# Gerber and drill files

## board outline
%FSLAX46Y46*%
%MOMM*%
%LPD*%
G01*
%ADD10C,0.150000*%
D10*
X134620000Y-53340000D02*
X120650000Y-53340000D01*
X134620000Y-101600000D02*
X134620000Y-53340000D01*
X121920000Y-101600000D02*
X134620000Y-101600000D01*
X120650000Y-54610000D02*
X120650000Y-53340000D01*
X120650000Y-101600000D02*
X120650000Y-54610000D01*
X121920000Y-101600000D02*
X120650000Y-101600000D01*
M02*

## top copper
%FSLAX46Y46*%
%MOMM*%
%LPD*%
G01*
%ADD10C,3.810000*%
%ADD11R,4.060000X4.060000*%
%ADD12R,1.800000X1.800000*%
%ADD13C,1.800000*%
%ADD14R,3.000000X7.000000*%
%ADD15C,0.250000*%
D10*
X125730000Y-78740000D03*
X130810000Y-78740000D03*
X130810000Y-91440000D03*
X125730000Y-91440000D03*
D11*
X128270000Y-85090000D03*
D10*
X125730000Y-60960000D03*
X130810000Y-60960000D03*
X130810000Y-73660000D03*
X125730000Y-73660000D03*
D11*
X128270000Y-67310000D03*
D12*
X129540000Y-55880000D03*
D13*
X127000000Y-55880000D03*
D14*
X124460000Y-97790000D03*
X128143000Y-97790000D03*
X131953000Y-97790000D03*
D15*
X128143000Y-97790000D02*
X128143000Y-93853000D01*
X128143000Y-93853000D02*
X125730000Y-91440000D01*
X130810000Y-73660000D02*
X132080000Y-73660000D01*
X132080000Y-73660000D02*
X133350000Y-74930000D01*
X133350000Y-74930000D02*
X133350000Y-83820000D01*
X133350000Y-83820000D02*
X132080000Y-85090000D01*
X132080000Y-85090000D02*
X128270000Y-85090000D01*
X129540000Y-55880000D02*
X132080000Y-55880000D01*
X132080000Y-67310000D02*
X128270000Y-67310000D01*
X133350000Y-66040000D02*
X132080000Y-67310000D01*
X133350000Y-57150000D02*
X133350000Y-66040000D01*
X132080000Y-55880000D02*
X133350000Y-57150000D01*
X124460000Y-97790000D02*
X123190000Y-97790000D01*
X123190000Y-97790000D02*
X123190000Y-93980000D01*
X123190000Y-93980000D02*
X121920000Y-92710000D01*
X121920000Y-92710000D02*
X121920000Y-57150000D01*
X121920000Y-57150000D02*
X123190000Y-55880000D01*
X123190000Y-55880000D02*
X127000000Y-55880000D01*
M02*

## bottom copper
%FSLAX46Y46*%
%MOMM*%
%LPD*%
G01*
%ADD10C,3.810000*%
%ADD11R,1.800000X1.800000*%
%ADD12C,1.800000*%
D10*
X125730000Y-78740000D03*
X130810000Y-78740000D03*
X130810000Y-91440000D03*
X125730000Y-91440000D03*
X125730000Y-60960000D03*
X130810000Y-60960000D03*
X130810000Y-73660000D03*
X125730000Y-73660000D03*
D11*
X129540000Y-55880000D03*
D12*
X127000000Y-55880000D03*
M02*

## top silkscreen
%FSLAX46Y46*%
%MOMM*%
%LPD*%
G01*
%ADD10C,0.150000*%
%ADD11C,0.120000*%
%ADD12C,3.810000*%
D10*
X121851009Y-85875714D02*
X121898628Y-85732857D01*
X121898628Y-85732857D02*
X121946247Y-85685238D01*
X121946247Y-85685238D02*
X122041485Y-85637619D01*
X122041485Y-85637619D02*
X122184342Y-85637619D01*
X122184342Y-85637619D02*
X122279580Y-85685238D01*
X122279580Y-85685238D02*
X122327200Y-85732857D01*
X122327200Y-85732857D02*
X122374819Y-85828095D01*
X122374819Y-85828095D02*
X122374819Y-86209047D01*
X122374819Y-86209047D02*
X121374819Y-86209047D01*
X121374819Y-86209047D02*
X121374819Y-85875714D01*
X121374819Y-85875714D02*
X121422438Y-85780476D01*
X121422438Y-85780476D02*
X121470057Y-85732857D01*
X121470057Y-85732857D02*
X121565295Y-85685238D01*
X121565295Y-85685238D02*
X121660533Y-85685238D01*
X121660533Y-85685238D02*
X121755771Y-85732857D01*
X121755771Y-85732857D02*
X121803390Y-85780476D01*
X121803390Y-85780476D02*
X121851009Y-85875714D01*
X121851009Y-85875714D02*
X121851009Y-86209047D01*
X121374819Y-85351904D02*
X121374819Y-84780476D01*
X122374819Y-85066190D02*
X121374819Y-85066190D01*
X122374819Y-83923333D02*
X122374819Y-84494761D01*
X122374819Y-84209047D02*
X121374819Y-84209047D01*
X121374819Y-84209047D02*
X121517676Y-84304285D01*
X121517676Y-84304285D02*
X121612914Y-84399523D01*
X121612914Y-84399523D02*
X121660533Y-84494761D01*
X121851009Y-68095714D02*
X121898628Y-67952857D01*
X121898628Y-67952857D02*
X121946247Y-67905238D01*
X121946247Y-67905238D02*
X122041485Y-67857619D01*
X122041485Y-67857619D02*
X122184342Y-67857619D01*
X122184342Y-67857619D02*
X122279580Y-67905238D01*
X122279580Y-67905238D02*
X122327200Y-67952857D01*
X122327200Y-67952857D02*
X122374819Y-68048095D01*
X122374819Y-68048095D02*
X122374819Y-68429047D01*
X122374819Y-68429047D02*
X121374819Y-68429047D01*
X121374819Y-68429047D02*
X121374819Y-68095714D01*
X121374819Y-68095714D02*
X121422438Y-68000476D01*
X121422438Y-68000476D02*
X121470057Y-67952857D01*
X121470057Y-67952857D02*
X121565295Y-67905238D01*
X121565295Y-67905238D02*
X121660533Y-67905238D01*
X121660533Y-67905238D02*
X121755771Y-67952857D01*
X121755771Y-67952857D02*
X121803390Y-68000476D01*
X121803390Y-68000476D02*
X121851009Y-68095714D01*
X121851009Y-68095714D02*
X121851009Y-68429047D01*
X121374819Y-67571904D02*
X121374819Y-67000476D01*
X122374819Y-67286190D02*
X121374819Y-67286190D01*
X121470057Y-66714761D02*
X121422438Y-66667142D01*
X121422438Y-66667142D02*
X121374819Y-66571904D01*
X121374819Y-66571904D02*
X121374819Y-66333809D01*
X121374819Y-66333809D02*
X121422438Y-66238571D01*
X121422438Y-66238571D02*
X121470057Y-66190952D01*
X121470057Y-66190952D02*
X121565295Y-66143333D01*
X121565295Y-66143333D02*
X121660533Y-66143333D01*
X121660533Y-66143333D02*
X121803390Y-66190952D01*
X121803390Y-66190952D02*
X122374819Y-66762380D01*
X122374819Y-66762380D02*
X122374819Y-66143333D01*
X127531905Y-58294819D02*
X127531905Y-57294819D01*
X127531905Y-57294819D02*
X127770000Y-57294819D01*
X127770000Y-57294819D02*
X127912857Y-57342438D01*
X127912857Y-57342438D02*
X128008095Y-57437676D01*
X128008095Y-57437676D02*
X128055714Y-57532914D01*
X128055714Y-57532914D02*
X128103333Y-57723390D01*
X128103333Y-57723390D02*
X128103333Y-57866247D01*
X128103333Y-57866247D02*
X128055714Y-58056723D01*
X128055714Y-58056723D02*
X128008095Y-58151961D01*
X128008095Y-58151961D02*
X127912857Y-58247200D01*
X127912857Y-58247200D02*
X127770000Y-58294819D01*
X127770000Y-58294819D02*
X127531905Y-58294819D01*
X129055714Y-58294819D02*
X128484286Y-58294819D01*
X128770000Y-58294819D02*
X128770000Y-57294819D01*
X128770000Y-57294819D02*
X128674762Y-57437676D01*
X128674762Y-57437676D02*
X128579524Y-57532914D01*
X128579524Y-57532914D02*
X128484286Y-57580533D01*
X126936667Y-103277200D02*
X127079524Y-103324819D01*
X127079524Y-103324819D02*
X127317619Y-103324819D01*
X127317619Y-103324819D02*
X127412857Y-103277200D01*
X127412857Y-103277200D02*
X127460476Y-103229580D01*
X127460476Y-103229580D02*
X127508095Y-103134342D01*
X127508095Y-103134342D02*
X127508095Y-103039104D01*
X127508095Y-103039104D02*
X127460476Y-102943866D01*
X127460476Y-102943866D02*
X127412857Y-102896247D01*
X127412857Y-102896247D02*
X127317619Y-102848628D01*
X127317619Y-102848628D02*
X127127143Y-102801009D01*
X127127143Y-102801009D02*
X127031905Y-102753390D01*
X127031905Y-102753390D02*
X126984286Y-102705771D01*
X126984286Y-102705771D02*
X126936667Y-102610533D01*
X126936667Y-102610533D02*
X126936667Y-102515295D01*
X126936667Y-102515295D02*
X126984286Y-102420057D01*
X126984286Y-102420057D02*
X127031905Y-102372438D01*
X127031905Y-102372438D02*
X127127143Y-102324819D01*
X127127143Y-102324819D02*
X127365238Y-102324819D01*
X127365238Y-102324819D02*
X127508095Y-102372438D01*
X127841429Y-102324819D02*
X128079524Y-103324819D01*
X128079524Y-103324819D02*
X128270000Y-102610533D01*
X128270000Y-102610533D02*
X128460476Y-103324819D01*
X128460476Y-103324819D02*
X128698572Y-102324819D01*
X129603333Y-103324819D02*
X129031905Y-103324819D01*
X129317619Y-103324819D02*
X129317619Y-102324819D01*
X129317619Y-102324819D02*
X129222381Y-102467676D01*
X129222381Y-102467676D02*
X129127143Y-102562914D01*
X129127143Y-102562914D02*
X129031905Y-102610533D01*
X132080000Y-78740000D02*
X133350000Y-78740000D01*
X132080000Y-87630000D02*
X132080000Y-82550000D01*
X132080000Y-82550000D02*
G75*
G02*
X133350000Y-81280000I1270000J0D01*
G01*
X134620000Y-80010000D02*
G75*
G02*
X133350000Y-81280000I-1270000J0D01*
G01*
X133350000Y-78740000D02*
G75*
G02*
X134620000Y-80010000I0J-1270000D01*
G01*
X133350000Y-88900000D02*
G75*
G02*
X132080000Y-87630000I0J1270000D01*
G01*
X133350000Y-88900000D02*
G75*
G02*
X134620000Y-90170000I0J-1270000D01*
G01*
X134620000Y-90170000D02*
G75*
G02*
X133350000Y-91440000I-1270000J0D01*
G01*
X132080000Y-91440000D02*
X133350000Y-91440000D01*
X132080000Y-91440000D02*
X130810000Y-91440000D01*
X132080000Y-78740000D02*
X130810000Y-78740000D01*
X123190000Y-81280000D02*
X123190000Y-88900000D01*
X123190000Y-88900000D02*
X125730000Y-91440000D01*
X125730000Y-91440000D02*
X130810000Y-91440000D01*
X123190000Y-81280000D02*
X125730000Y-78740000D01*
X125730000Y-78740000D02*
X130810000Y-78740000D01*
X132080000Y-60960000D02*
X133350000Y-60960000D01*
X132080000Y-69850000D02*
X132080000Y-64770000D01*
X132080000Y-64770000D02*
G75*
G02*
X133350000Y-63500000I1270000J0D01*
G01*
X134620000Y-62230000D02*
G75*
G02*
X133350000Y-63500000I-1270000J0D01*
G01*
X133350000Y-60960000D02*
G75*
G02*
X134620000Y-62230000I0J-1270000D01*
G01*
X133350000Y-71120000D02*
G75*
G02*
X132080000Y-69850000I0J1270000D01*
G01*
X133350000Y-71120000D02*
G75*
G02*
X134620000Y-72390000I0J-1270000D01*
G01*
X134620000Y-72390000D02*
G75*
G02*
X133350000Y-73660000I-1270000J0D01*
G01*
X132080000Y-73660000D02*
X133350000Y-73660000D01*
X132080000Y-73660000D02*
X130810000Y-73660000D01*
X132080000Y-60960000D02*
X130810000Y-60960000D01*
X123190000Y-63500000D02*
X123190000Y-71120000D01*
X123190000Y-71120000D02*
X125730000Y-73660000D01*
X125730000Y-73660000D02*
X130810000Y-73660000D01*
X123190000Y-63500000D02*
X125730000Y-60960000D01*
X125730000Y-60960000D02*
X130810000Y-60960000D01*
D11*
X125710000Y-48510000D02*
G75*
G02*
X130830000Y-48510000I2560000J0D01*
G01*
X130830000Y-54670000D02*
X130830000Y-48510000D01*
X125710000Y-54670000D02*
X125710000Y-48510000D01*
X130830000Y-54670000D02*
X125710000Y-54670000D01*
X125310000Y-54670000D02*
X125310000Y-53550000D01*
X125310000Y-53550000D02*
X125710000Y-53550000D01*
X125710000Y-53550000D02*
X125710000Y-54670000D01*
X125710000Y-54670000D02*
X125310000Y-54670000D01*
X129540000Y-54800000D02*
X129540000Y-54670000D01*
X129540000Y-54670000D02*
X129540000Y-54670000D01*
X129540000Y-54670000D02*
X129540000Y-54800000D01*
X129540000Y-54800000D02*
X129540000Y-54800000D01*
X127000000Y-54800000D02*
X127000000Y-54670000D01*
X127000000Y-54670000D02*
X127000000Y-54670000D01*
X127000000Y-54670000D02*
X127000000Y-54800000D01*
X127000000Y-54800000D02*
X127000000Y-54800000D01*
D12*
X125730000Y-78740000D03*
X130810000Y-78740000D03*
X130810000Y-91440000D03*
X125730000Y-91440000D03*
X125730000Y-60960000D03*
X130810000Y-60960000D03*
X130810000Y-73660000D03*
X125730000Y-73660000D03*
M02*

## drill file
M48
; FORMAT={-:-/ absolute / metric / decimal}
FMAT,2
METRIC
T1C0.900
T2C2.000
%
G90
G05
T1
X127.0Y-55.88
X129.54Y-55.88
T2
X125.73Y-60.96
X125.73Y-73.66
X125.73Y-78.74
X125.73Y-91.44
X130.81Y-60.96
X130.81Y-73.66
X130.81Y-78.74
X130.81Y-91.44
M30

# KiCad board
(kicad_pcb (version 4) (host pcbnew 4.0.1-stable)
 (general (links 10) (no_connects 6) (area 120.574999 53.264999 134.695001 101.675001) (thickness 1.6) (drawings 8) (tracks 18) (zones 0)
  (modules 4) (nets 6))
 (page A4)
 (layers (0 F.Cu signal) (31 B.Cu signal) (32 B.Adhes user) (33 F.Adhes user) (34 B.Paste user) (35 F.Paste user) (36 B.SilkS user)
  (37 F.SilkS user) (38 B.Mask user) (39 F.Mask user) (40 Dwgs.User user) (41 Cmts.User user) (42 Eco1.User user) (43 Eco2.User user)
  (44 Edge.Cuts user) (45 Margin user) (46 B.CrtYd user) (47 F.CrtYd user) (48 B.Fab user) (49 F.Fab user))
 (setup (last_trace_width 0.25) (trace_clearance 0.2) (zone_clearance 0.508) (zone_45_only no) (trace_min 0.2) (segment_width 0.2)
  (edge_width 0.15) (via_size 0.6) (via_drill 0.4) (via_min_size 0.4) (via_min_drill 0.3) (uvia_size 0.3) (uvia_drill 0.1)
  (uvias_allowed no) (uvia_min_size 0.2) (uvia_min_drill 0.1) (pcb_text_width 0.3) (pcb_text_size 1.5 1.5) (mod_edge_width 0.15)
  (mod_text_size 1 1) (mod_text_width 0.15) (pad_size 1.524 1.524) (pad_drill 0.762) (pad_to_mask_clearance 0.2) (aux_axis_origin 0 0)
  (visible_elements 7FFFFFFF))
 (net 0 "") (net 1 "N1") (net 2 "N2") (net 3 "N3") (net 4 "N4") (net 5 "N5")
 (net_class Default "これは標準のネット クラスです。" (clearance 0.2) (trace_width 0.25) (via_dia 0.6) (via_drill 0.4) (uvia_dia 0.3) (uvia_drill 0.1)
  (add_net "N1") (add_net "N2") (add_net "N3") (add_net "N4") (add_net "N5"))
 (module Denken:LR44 (layer F.Cu) (at 128.27 85.09 270)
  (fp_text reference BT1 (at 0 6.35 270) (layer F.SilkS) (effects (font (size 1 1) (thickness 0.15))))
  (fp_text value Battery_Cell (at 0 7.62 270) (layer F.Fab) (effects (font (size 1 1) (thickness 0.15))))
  (fp_line (start -6.35 -3.81) (end -6.35 -5.08) (layer F.SilkS) (width 0.15))
  (fp_line (start 2.54 -3.81) (end -2.54 -3.81) (layer F.SilkS) (width 0.15))
  (fp_arc (start -2.54 -5.08) (end -2.54 -3.81) (angle 90) (layer F.SilkS) (width 0.15))
  (fp_arc (start -5.08 -5.08) (end -5.08 -6.35) (angle 90) (layer F.SilkS) (width 0.15))
  (fp_arc (start -5.08 -5.08) (end -6.35 -5.08) (angle 90) (layer F.SilkS) (width 0.15))
  (fp_arc (start 2.54 -5.08) (end 3.81 -5.08) (angle 90) (layer F.SilkS) (width 0.15))
  (fp_arc (start 5.08 -5.08) (end 3.81 -5.08) (angle 90) (layer F.SilkS) (width 0.15))
  (fp_arc (start 5.08 -5.08) (end 5.08 -6.35) (angle 90) (layer F.SilkS) (width 0.15))
  (fp_line (start 6.35 -3.81) (end 6.35 -5.08) (layer F.SilkS) (width 0.15))
  (fp_line (start 6.35 -3.81) (end 6.35 -2.54) (layer F.SilkS) (width 0.15))
  (fp_line (start -6.35 -3.81) (end -6.35 -2.54) (layer F.SilkS) (width 0.15))
  (fp_line (start -3.81 5.08) (end 3.81 5.08) (layer F.SilkS) (width 0.15))
  (fp_line (start 3.81 5.08) (end 6.35 2.54) (layer F.SilkS) (width 0.15))
  (fp_line (start 6.35 2.54) (end 6.35 -2.54) (layer F.SilkS) (width 0.15))
  (fp_line (start -3.81 5.08) (end -6.35 2.54) (layer F.SilkS) (width 0.15))
  (fp_line (start -6.35 2.54) (end -6.35 -2.54) (layer F.SilkS) (width 0.15))
  (pad 1 thru_hole circle (at -6.35 2.54 270) (size 3.81 3.81) (drill 2) (layers *.Cu *.Mask F.SilkS) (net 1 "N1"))
  (pad 1 thru_hole circle (at -6.35 -2.54 270) (size 3.81 3.81) (drill 2) (layers *.Cu *.Mask F.SilkS) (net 1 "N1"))
  (pad 1 thru_hole circle (at 6.35 -2.54 270) (size 3.81 3.81) (drill 2) (layers *.Cu *.Mask F.SilkS) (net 1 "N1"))
  (pad 1 thru_hole circle (at 6.35 2.54 270) (size 3.81 3.81) (drill 2) (layers *.Cu *.Mask F.SilkS) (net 1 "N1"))
  (pad 2 smd rect (at 0 0 270) (size 4.06 4.06) (layers F.Cu F.Paste F.Mask) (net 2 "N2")))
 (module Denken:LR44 (layer F.Cu) (at 128.27 67.31 270)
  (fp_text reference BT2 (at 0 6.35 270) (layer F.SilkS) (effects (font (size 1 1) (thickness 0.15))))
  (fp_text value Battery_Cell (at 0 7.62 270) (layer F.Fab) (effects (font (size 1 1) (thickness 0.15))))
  (fp_line (start -6.35 -3.81) (end -6.35 -5.08) (layer F.SilkS) (width 0.15))
  (fp_line (start 2.54 -3.81) (end -2.54 -3.81) (layer F.SilkS) (width 0.15))
  (fp_arc (start -2.54 -5.08) (end -2.54 -3.81) (angle 90) (layer F.SilkS) (width 0.15))
  (fp_arc (start -5.08 -5.08) (end -5.08 -6.35) (angle 90) (layer F.SilkS) (width 0.15))
  (fp_arc (start -5.08 -5.08) (end -6.35 -5.08) (angle 90) (layer F.SilkS) (width 0.15))
  (fp_arc (start 2.54 -5.08) (end 3.81 -5.08) (angle 90) (layer F.SilkS) (width 0.15))
  (fp_arc (start 5.08 -5.08) (end 3.81 -5.08) (angle 90) (layer F.SilkS) (width 0.15))
  (fp_arc (start 5.08 -5.08) (end 5.08 -6.35) (angle 90) (layer F.SilkS) (width 0.15))
  (fp_line (start 6.35 -3.81) (end 6.35 -5.08) (layer F.SilkS) (width 0.15))
  (fp_line (start 6.35 -3.81) (end 6.35 -2.54) (layer F.SilkS) (width 0.15))
  (fp_line (start -6.35 -3.81) (end -6.35 -2.54) (layer F.SilkS) (width 0.15))
  (fp_line (start -3.81 5.08) (end 3.81 5.08) (layer F.SilkS) (width 0.15))
  (fp_line (start 3.81 5.08) (end 6.35 2.54) (layer F.SilkS) (width 0.15))
  (fp_line (start 6.35 2.54) (end 6.35 -2.54) (layer F.SilkS) (width 0.15))
  (fp_line (start -3.81 5.08) (end -6.35 2.54) (layer F.SilkS) (width 0.15))
  (fp_line (start -6.35 2.54) (end -6.35 -2.54) (layer F.SilkS) (width 0.15))
  (pad 1 thru_hole circle (at -6.35 2.54 270) (size 3.81 3.81) (drill 2) (layers *.Cu *.Mask F.SilkS) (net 2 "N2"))
  (pad 1 thru_hole circle (at -6.35 -2.54 270) (size 3.81 3.81) (drill 2) (layers *.Cu *.Mask F.SilkS) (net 2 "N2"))
  (pad 1 thru_hole circle (at 6.35 -2.54 270) (size 3.81 3.81) (drill 2) (layers *.Cu *.Mask F.SilkS) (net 2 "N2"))
  (pad 1 thru_hole circle (at 6.35 2.54 270) (size 3.81 3.81) (drill 2) (layers *.Cu *.Mask F.SilkS) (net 2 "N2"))
  (pad 2 smd rect (at 0 0 270) (size 4.06 4.06) (layers F.Cu F.Paste F.Mask) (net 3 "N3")))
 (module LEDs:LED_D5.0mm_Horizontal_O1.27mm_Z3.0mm (layer F.Cu) (at 129.54 55.88 180)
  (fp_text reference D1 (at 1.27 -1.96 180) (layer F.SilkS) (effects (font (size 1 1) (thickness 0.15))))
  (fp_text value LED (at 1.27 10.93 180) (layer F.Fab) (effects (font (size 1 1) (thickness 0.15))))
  (fp_arc (start 1.27 7.37) (end -1.29 7.37) (angle -180) (layer F.SilkS) (width 0.12))
  (fp_line (start -1.29 1.21) (end -1.29 7.37) (layer F.SilkS) (width 0.12))
  (fp_line (start 3.83 1.21) (end 3.83 7.37) (layer F.SilkS) (width 0.12))
  (fp_line (start -1.29 1.21) (end 3.83 1.21) (layer F.SilkS) (width 0.12))
  (fp_line (start 4.23 1.21) (end 4.23 2.33) (layer F.SilkS) (width 0.12))
  (fp_line (start 4.23 2.33) (end 3.83 2.33) (layer F.SilkS) (width 0.12))
  (fp_line (start 3.83 2.33) (end 3.83 1.21) (layer F.SilkS) (width 0.12))
  (fp_line (start 3.83 1.21) (end 4.23 1.21) (layer F.SilkS) (width 0.12))
  (fp_line (start 0 1.08) (end 0 1.21) (layer F.SilkS) (width 0.12))
  (fp_line (start 0 1.21) (end 0 1.21) (layer F.SilkS) (width 0.12))
  (fp_line (start 0 1.21) (end 0 1.08) (layer F.SilkS) (width 0.12))
  (fp_line (start 0 1.08) (end 0 1.08) (layer F.SilkS) (width 0.12))
  (fp_line (start 2.54 1.08) (end 2.54 1.21) (layer F.SilkS) (width 0.12))
  (fp_line (start 2.54 1.21) (end 2.54 1.21) (layer F.SilkS) (width 0.12))
  (fp_line (start 2.54 1.21) (end 2.54 1.08) (layer F.SilkS) (width 0.12))
  (fp_line (start 2.54 1.08) (end 2.54 1.08) (layer F.SilkS) (width 0.12))
  (pad 1 thru_hole rect (at 0 0 180) (size 1.8 1.8) (drill 0.9) (layers *.Cu *.Mask) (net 3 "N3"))
  (pad 2 thru_hole circle (at 2.54 0 180) (size 1.8 1.8) (drill 0.9) (layers *.Cu *.Mask) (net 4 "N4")))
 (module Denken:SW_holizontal (layer F.Cu) (at 128.27 97.79)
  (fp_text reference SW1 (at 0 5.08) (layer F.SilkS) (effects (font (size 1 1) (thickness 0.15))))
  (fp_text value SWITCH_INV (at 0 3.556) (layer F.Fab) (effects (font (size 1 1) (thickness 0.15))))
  (pad 1 smd rect (at -3.81 0) (size 3 7) (layers F.Cu F.Paste F.Mask) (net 4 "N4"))
  (pad 2 smd rect (at -0.127 0) (size 3 7) (layers F.Cu F.Paste F.Mask) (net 1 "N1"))
  (pad 3 smd rect (at 3.683 0) (size 3 7) (layers F.Cu F.Paste F.Mask) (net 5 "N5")))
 (gr_line (start 134.62 53.34) (end 120.65 53.34) (angle 90) (layer Edge.Cuts) (width 0.15))
 (gr_line (start 134.62 101.6) (end 134.62 53.34) (angle 90) (layer Edge.Cuts) (width 0.15))
 (gr_line (start 121.92 101.6) (end 134.62 101.6) (angle 90) (layer Edge.Cuts) (width 0.15))
 (gr_line (start 120.65 54.61) (end 120.65 53.34) (angle 90) (layer Edge.Cuts) (width 0.15))
 (gr_line (start 120.65 101.6) (end 120.65 54.61) (angle 90) (layer Edge.Cuts) (width 0.15))
 (gr_line (start 121.92 101.6) (end 120.65 101.6) (angle 90) (layer Edge.Cuts) (width 0.15))
 (segment (start 128.143 97.79) (end 128.143 93.853) (width 0.25) (layer F.Cu) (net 1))
 (segment (start 128.143 93.853) (end 125.73 91.44) (width 0.25) (layer F.Cu) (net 1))
 (segment (start 130.81 73.66) (end 132.08 73.66) (width 0.25) (layer F.Cu) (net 2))
 (segment (start 132.08 73.66) (end 133.35 74.93) (width 0.25) (layer F.Cu) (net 2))
 (segment (start 133.35 74.93) (end 133.35 83.82) (width 0.25) (layer F.Cu) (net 2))
 (segment (start 133.35 83.82) (end 132.08 85.09) (width 0.25) (layer F.Cu) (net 2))
 (segment (start 132.08 85.09) (end 128.27 85.09) (width 0.25) (layer F.Cu) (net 2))
 (segment (start 129.54 55.88) (end 132.08 55.88) (width 0.25) (layer F.Cu) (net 3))
 (segment (start 132.08 67.31) (end 128.27 67.31) (width 0.25) (layer F.Cu) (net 3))
 (segment (start 133.35 66.04) (end 132.08 67.31) (width 0.25) (layer F.Cu) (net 3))
 (segment (start 133.35 57.15) (end 133.35 66.04) (width 0.25) (layer F.Cu) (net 3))
 (segment (start 132.08 55.88) (end 133.35 57.15) (width 0.25) (layer F.Cu) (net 3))
 (segment (start 124.46 97.79) (end 123.19 97.79) (width 0.25) (layer F.Cu) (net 4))
 (segment (start 123.19 97.79) (end 123.19 93.98) (width 0.25) (layer F.Cu) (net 4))
 (segment (start 123.19 93.98) (end 121.92 92.71) (width 0.25) (layer F.Cu) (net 4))
 (segment (start 121.92 92.71) (end 121.92 57.15) (width 0.25) (layer F.Cu) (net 4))
 (segment (start 121.92 57.15) (end 123.19 55.88) (width 0.25) (layer F.Cu) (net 4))
 (segment (start 123.19 55.88) (end 127 55.88) (width 0.25) (layer F.Cu) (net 4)))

